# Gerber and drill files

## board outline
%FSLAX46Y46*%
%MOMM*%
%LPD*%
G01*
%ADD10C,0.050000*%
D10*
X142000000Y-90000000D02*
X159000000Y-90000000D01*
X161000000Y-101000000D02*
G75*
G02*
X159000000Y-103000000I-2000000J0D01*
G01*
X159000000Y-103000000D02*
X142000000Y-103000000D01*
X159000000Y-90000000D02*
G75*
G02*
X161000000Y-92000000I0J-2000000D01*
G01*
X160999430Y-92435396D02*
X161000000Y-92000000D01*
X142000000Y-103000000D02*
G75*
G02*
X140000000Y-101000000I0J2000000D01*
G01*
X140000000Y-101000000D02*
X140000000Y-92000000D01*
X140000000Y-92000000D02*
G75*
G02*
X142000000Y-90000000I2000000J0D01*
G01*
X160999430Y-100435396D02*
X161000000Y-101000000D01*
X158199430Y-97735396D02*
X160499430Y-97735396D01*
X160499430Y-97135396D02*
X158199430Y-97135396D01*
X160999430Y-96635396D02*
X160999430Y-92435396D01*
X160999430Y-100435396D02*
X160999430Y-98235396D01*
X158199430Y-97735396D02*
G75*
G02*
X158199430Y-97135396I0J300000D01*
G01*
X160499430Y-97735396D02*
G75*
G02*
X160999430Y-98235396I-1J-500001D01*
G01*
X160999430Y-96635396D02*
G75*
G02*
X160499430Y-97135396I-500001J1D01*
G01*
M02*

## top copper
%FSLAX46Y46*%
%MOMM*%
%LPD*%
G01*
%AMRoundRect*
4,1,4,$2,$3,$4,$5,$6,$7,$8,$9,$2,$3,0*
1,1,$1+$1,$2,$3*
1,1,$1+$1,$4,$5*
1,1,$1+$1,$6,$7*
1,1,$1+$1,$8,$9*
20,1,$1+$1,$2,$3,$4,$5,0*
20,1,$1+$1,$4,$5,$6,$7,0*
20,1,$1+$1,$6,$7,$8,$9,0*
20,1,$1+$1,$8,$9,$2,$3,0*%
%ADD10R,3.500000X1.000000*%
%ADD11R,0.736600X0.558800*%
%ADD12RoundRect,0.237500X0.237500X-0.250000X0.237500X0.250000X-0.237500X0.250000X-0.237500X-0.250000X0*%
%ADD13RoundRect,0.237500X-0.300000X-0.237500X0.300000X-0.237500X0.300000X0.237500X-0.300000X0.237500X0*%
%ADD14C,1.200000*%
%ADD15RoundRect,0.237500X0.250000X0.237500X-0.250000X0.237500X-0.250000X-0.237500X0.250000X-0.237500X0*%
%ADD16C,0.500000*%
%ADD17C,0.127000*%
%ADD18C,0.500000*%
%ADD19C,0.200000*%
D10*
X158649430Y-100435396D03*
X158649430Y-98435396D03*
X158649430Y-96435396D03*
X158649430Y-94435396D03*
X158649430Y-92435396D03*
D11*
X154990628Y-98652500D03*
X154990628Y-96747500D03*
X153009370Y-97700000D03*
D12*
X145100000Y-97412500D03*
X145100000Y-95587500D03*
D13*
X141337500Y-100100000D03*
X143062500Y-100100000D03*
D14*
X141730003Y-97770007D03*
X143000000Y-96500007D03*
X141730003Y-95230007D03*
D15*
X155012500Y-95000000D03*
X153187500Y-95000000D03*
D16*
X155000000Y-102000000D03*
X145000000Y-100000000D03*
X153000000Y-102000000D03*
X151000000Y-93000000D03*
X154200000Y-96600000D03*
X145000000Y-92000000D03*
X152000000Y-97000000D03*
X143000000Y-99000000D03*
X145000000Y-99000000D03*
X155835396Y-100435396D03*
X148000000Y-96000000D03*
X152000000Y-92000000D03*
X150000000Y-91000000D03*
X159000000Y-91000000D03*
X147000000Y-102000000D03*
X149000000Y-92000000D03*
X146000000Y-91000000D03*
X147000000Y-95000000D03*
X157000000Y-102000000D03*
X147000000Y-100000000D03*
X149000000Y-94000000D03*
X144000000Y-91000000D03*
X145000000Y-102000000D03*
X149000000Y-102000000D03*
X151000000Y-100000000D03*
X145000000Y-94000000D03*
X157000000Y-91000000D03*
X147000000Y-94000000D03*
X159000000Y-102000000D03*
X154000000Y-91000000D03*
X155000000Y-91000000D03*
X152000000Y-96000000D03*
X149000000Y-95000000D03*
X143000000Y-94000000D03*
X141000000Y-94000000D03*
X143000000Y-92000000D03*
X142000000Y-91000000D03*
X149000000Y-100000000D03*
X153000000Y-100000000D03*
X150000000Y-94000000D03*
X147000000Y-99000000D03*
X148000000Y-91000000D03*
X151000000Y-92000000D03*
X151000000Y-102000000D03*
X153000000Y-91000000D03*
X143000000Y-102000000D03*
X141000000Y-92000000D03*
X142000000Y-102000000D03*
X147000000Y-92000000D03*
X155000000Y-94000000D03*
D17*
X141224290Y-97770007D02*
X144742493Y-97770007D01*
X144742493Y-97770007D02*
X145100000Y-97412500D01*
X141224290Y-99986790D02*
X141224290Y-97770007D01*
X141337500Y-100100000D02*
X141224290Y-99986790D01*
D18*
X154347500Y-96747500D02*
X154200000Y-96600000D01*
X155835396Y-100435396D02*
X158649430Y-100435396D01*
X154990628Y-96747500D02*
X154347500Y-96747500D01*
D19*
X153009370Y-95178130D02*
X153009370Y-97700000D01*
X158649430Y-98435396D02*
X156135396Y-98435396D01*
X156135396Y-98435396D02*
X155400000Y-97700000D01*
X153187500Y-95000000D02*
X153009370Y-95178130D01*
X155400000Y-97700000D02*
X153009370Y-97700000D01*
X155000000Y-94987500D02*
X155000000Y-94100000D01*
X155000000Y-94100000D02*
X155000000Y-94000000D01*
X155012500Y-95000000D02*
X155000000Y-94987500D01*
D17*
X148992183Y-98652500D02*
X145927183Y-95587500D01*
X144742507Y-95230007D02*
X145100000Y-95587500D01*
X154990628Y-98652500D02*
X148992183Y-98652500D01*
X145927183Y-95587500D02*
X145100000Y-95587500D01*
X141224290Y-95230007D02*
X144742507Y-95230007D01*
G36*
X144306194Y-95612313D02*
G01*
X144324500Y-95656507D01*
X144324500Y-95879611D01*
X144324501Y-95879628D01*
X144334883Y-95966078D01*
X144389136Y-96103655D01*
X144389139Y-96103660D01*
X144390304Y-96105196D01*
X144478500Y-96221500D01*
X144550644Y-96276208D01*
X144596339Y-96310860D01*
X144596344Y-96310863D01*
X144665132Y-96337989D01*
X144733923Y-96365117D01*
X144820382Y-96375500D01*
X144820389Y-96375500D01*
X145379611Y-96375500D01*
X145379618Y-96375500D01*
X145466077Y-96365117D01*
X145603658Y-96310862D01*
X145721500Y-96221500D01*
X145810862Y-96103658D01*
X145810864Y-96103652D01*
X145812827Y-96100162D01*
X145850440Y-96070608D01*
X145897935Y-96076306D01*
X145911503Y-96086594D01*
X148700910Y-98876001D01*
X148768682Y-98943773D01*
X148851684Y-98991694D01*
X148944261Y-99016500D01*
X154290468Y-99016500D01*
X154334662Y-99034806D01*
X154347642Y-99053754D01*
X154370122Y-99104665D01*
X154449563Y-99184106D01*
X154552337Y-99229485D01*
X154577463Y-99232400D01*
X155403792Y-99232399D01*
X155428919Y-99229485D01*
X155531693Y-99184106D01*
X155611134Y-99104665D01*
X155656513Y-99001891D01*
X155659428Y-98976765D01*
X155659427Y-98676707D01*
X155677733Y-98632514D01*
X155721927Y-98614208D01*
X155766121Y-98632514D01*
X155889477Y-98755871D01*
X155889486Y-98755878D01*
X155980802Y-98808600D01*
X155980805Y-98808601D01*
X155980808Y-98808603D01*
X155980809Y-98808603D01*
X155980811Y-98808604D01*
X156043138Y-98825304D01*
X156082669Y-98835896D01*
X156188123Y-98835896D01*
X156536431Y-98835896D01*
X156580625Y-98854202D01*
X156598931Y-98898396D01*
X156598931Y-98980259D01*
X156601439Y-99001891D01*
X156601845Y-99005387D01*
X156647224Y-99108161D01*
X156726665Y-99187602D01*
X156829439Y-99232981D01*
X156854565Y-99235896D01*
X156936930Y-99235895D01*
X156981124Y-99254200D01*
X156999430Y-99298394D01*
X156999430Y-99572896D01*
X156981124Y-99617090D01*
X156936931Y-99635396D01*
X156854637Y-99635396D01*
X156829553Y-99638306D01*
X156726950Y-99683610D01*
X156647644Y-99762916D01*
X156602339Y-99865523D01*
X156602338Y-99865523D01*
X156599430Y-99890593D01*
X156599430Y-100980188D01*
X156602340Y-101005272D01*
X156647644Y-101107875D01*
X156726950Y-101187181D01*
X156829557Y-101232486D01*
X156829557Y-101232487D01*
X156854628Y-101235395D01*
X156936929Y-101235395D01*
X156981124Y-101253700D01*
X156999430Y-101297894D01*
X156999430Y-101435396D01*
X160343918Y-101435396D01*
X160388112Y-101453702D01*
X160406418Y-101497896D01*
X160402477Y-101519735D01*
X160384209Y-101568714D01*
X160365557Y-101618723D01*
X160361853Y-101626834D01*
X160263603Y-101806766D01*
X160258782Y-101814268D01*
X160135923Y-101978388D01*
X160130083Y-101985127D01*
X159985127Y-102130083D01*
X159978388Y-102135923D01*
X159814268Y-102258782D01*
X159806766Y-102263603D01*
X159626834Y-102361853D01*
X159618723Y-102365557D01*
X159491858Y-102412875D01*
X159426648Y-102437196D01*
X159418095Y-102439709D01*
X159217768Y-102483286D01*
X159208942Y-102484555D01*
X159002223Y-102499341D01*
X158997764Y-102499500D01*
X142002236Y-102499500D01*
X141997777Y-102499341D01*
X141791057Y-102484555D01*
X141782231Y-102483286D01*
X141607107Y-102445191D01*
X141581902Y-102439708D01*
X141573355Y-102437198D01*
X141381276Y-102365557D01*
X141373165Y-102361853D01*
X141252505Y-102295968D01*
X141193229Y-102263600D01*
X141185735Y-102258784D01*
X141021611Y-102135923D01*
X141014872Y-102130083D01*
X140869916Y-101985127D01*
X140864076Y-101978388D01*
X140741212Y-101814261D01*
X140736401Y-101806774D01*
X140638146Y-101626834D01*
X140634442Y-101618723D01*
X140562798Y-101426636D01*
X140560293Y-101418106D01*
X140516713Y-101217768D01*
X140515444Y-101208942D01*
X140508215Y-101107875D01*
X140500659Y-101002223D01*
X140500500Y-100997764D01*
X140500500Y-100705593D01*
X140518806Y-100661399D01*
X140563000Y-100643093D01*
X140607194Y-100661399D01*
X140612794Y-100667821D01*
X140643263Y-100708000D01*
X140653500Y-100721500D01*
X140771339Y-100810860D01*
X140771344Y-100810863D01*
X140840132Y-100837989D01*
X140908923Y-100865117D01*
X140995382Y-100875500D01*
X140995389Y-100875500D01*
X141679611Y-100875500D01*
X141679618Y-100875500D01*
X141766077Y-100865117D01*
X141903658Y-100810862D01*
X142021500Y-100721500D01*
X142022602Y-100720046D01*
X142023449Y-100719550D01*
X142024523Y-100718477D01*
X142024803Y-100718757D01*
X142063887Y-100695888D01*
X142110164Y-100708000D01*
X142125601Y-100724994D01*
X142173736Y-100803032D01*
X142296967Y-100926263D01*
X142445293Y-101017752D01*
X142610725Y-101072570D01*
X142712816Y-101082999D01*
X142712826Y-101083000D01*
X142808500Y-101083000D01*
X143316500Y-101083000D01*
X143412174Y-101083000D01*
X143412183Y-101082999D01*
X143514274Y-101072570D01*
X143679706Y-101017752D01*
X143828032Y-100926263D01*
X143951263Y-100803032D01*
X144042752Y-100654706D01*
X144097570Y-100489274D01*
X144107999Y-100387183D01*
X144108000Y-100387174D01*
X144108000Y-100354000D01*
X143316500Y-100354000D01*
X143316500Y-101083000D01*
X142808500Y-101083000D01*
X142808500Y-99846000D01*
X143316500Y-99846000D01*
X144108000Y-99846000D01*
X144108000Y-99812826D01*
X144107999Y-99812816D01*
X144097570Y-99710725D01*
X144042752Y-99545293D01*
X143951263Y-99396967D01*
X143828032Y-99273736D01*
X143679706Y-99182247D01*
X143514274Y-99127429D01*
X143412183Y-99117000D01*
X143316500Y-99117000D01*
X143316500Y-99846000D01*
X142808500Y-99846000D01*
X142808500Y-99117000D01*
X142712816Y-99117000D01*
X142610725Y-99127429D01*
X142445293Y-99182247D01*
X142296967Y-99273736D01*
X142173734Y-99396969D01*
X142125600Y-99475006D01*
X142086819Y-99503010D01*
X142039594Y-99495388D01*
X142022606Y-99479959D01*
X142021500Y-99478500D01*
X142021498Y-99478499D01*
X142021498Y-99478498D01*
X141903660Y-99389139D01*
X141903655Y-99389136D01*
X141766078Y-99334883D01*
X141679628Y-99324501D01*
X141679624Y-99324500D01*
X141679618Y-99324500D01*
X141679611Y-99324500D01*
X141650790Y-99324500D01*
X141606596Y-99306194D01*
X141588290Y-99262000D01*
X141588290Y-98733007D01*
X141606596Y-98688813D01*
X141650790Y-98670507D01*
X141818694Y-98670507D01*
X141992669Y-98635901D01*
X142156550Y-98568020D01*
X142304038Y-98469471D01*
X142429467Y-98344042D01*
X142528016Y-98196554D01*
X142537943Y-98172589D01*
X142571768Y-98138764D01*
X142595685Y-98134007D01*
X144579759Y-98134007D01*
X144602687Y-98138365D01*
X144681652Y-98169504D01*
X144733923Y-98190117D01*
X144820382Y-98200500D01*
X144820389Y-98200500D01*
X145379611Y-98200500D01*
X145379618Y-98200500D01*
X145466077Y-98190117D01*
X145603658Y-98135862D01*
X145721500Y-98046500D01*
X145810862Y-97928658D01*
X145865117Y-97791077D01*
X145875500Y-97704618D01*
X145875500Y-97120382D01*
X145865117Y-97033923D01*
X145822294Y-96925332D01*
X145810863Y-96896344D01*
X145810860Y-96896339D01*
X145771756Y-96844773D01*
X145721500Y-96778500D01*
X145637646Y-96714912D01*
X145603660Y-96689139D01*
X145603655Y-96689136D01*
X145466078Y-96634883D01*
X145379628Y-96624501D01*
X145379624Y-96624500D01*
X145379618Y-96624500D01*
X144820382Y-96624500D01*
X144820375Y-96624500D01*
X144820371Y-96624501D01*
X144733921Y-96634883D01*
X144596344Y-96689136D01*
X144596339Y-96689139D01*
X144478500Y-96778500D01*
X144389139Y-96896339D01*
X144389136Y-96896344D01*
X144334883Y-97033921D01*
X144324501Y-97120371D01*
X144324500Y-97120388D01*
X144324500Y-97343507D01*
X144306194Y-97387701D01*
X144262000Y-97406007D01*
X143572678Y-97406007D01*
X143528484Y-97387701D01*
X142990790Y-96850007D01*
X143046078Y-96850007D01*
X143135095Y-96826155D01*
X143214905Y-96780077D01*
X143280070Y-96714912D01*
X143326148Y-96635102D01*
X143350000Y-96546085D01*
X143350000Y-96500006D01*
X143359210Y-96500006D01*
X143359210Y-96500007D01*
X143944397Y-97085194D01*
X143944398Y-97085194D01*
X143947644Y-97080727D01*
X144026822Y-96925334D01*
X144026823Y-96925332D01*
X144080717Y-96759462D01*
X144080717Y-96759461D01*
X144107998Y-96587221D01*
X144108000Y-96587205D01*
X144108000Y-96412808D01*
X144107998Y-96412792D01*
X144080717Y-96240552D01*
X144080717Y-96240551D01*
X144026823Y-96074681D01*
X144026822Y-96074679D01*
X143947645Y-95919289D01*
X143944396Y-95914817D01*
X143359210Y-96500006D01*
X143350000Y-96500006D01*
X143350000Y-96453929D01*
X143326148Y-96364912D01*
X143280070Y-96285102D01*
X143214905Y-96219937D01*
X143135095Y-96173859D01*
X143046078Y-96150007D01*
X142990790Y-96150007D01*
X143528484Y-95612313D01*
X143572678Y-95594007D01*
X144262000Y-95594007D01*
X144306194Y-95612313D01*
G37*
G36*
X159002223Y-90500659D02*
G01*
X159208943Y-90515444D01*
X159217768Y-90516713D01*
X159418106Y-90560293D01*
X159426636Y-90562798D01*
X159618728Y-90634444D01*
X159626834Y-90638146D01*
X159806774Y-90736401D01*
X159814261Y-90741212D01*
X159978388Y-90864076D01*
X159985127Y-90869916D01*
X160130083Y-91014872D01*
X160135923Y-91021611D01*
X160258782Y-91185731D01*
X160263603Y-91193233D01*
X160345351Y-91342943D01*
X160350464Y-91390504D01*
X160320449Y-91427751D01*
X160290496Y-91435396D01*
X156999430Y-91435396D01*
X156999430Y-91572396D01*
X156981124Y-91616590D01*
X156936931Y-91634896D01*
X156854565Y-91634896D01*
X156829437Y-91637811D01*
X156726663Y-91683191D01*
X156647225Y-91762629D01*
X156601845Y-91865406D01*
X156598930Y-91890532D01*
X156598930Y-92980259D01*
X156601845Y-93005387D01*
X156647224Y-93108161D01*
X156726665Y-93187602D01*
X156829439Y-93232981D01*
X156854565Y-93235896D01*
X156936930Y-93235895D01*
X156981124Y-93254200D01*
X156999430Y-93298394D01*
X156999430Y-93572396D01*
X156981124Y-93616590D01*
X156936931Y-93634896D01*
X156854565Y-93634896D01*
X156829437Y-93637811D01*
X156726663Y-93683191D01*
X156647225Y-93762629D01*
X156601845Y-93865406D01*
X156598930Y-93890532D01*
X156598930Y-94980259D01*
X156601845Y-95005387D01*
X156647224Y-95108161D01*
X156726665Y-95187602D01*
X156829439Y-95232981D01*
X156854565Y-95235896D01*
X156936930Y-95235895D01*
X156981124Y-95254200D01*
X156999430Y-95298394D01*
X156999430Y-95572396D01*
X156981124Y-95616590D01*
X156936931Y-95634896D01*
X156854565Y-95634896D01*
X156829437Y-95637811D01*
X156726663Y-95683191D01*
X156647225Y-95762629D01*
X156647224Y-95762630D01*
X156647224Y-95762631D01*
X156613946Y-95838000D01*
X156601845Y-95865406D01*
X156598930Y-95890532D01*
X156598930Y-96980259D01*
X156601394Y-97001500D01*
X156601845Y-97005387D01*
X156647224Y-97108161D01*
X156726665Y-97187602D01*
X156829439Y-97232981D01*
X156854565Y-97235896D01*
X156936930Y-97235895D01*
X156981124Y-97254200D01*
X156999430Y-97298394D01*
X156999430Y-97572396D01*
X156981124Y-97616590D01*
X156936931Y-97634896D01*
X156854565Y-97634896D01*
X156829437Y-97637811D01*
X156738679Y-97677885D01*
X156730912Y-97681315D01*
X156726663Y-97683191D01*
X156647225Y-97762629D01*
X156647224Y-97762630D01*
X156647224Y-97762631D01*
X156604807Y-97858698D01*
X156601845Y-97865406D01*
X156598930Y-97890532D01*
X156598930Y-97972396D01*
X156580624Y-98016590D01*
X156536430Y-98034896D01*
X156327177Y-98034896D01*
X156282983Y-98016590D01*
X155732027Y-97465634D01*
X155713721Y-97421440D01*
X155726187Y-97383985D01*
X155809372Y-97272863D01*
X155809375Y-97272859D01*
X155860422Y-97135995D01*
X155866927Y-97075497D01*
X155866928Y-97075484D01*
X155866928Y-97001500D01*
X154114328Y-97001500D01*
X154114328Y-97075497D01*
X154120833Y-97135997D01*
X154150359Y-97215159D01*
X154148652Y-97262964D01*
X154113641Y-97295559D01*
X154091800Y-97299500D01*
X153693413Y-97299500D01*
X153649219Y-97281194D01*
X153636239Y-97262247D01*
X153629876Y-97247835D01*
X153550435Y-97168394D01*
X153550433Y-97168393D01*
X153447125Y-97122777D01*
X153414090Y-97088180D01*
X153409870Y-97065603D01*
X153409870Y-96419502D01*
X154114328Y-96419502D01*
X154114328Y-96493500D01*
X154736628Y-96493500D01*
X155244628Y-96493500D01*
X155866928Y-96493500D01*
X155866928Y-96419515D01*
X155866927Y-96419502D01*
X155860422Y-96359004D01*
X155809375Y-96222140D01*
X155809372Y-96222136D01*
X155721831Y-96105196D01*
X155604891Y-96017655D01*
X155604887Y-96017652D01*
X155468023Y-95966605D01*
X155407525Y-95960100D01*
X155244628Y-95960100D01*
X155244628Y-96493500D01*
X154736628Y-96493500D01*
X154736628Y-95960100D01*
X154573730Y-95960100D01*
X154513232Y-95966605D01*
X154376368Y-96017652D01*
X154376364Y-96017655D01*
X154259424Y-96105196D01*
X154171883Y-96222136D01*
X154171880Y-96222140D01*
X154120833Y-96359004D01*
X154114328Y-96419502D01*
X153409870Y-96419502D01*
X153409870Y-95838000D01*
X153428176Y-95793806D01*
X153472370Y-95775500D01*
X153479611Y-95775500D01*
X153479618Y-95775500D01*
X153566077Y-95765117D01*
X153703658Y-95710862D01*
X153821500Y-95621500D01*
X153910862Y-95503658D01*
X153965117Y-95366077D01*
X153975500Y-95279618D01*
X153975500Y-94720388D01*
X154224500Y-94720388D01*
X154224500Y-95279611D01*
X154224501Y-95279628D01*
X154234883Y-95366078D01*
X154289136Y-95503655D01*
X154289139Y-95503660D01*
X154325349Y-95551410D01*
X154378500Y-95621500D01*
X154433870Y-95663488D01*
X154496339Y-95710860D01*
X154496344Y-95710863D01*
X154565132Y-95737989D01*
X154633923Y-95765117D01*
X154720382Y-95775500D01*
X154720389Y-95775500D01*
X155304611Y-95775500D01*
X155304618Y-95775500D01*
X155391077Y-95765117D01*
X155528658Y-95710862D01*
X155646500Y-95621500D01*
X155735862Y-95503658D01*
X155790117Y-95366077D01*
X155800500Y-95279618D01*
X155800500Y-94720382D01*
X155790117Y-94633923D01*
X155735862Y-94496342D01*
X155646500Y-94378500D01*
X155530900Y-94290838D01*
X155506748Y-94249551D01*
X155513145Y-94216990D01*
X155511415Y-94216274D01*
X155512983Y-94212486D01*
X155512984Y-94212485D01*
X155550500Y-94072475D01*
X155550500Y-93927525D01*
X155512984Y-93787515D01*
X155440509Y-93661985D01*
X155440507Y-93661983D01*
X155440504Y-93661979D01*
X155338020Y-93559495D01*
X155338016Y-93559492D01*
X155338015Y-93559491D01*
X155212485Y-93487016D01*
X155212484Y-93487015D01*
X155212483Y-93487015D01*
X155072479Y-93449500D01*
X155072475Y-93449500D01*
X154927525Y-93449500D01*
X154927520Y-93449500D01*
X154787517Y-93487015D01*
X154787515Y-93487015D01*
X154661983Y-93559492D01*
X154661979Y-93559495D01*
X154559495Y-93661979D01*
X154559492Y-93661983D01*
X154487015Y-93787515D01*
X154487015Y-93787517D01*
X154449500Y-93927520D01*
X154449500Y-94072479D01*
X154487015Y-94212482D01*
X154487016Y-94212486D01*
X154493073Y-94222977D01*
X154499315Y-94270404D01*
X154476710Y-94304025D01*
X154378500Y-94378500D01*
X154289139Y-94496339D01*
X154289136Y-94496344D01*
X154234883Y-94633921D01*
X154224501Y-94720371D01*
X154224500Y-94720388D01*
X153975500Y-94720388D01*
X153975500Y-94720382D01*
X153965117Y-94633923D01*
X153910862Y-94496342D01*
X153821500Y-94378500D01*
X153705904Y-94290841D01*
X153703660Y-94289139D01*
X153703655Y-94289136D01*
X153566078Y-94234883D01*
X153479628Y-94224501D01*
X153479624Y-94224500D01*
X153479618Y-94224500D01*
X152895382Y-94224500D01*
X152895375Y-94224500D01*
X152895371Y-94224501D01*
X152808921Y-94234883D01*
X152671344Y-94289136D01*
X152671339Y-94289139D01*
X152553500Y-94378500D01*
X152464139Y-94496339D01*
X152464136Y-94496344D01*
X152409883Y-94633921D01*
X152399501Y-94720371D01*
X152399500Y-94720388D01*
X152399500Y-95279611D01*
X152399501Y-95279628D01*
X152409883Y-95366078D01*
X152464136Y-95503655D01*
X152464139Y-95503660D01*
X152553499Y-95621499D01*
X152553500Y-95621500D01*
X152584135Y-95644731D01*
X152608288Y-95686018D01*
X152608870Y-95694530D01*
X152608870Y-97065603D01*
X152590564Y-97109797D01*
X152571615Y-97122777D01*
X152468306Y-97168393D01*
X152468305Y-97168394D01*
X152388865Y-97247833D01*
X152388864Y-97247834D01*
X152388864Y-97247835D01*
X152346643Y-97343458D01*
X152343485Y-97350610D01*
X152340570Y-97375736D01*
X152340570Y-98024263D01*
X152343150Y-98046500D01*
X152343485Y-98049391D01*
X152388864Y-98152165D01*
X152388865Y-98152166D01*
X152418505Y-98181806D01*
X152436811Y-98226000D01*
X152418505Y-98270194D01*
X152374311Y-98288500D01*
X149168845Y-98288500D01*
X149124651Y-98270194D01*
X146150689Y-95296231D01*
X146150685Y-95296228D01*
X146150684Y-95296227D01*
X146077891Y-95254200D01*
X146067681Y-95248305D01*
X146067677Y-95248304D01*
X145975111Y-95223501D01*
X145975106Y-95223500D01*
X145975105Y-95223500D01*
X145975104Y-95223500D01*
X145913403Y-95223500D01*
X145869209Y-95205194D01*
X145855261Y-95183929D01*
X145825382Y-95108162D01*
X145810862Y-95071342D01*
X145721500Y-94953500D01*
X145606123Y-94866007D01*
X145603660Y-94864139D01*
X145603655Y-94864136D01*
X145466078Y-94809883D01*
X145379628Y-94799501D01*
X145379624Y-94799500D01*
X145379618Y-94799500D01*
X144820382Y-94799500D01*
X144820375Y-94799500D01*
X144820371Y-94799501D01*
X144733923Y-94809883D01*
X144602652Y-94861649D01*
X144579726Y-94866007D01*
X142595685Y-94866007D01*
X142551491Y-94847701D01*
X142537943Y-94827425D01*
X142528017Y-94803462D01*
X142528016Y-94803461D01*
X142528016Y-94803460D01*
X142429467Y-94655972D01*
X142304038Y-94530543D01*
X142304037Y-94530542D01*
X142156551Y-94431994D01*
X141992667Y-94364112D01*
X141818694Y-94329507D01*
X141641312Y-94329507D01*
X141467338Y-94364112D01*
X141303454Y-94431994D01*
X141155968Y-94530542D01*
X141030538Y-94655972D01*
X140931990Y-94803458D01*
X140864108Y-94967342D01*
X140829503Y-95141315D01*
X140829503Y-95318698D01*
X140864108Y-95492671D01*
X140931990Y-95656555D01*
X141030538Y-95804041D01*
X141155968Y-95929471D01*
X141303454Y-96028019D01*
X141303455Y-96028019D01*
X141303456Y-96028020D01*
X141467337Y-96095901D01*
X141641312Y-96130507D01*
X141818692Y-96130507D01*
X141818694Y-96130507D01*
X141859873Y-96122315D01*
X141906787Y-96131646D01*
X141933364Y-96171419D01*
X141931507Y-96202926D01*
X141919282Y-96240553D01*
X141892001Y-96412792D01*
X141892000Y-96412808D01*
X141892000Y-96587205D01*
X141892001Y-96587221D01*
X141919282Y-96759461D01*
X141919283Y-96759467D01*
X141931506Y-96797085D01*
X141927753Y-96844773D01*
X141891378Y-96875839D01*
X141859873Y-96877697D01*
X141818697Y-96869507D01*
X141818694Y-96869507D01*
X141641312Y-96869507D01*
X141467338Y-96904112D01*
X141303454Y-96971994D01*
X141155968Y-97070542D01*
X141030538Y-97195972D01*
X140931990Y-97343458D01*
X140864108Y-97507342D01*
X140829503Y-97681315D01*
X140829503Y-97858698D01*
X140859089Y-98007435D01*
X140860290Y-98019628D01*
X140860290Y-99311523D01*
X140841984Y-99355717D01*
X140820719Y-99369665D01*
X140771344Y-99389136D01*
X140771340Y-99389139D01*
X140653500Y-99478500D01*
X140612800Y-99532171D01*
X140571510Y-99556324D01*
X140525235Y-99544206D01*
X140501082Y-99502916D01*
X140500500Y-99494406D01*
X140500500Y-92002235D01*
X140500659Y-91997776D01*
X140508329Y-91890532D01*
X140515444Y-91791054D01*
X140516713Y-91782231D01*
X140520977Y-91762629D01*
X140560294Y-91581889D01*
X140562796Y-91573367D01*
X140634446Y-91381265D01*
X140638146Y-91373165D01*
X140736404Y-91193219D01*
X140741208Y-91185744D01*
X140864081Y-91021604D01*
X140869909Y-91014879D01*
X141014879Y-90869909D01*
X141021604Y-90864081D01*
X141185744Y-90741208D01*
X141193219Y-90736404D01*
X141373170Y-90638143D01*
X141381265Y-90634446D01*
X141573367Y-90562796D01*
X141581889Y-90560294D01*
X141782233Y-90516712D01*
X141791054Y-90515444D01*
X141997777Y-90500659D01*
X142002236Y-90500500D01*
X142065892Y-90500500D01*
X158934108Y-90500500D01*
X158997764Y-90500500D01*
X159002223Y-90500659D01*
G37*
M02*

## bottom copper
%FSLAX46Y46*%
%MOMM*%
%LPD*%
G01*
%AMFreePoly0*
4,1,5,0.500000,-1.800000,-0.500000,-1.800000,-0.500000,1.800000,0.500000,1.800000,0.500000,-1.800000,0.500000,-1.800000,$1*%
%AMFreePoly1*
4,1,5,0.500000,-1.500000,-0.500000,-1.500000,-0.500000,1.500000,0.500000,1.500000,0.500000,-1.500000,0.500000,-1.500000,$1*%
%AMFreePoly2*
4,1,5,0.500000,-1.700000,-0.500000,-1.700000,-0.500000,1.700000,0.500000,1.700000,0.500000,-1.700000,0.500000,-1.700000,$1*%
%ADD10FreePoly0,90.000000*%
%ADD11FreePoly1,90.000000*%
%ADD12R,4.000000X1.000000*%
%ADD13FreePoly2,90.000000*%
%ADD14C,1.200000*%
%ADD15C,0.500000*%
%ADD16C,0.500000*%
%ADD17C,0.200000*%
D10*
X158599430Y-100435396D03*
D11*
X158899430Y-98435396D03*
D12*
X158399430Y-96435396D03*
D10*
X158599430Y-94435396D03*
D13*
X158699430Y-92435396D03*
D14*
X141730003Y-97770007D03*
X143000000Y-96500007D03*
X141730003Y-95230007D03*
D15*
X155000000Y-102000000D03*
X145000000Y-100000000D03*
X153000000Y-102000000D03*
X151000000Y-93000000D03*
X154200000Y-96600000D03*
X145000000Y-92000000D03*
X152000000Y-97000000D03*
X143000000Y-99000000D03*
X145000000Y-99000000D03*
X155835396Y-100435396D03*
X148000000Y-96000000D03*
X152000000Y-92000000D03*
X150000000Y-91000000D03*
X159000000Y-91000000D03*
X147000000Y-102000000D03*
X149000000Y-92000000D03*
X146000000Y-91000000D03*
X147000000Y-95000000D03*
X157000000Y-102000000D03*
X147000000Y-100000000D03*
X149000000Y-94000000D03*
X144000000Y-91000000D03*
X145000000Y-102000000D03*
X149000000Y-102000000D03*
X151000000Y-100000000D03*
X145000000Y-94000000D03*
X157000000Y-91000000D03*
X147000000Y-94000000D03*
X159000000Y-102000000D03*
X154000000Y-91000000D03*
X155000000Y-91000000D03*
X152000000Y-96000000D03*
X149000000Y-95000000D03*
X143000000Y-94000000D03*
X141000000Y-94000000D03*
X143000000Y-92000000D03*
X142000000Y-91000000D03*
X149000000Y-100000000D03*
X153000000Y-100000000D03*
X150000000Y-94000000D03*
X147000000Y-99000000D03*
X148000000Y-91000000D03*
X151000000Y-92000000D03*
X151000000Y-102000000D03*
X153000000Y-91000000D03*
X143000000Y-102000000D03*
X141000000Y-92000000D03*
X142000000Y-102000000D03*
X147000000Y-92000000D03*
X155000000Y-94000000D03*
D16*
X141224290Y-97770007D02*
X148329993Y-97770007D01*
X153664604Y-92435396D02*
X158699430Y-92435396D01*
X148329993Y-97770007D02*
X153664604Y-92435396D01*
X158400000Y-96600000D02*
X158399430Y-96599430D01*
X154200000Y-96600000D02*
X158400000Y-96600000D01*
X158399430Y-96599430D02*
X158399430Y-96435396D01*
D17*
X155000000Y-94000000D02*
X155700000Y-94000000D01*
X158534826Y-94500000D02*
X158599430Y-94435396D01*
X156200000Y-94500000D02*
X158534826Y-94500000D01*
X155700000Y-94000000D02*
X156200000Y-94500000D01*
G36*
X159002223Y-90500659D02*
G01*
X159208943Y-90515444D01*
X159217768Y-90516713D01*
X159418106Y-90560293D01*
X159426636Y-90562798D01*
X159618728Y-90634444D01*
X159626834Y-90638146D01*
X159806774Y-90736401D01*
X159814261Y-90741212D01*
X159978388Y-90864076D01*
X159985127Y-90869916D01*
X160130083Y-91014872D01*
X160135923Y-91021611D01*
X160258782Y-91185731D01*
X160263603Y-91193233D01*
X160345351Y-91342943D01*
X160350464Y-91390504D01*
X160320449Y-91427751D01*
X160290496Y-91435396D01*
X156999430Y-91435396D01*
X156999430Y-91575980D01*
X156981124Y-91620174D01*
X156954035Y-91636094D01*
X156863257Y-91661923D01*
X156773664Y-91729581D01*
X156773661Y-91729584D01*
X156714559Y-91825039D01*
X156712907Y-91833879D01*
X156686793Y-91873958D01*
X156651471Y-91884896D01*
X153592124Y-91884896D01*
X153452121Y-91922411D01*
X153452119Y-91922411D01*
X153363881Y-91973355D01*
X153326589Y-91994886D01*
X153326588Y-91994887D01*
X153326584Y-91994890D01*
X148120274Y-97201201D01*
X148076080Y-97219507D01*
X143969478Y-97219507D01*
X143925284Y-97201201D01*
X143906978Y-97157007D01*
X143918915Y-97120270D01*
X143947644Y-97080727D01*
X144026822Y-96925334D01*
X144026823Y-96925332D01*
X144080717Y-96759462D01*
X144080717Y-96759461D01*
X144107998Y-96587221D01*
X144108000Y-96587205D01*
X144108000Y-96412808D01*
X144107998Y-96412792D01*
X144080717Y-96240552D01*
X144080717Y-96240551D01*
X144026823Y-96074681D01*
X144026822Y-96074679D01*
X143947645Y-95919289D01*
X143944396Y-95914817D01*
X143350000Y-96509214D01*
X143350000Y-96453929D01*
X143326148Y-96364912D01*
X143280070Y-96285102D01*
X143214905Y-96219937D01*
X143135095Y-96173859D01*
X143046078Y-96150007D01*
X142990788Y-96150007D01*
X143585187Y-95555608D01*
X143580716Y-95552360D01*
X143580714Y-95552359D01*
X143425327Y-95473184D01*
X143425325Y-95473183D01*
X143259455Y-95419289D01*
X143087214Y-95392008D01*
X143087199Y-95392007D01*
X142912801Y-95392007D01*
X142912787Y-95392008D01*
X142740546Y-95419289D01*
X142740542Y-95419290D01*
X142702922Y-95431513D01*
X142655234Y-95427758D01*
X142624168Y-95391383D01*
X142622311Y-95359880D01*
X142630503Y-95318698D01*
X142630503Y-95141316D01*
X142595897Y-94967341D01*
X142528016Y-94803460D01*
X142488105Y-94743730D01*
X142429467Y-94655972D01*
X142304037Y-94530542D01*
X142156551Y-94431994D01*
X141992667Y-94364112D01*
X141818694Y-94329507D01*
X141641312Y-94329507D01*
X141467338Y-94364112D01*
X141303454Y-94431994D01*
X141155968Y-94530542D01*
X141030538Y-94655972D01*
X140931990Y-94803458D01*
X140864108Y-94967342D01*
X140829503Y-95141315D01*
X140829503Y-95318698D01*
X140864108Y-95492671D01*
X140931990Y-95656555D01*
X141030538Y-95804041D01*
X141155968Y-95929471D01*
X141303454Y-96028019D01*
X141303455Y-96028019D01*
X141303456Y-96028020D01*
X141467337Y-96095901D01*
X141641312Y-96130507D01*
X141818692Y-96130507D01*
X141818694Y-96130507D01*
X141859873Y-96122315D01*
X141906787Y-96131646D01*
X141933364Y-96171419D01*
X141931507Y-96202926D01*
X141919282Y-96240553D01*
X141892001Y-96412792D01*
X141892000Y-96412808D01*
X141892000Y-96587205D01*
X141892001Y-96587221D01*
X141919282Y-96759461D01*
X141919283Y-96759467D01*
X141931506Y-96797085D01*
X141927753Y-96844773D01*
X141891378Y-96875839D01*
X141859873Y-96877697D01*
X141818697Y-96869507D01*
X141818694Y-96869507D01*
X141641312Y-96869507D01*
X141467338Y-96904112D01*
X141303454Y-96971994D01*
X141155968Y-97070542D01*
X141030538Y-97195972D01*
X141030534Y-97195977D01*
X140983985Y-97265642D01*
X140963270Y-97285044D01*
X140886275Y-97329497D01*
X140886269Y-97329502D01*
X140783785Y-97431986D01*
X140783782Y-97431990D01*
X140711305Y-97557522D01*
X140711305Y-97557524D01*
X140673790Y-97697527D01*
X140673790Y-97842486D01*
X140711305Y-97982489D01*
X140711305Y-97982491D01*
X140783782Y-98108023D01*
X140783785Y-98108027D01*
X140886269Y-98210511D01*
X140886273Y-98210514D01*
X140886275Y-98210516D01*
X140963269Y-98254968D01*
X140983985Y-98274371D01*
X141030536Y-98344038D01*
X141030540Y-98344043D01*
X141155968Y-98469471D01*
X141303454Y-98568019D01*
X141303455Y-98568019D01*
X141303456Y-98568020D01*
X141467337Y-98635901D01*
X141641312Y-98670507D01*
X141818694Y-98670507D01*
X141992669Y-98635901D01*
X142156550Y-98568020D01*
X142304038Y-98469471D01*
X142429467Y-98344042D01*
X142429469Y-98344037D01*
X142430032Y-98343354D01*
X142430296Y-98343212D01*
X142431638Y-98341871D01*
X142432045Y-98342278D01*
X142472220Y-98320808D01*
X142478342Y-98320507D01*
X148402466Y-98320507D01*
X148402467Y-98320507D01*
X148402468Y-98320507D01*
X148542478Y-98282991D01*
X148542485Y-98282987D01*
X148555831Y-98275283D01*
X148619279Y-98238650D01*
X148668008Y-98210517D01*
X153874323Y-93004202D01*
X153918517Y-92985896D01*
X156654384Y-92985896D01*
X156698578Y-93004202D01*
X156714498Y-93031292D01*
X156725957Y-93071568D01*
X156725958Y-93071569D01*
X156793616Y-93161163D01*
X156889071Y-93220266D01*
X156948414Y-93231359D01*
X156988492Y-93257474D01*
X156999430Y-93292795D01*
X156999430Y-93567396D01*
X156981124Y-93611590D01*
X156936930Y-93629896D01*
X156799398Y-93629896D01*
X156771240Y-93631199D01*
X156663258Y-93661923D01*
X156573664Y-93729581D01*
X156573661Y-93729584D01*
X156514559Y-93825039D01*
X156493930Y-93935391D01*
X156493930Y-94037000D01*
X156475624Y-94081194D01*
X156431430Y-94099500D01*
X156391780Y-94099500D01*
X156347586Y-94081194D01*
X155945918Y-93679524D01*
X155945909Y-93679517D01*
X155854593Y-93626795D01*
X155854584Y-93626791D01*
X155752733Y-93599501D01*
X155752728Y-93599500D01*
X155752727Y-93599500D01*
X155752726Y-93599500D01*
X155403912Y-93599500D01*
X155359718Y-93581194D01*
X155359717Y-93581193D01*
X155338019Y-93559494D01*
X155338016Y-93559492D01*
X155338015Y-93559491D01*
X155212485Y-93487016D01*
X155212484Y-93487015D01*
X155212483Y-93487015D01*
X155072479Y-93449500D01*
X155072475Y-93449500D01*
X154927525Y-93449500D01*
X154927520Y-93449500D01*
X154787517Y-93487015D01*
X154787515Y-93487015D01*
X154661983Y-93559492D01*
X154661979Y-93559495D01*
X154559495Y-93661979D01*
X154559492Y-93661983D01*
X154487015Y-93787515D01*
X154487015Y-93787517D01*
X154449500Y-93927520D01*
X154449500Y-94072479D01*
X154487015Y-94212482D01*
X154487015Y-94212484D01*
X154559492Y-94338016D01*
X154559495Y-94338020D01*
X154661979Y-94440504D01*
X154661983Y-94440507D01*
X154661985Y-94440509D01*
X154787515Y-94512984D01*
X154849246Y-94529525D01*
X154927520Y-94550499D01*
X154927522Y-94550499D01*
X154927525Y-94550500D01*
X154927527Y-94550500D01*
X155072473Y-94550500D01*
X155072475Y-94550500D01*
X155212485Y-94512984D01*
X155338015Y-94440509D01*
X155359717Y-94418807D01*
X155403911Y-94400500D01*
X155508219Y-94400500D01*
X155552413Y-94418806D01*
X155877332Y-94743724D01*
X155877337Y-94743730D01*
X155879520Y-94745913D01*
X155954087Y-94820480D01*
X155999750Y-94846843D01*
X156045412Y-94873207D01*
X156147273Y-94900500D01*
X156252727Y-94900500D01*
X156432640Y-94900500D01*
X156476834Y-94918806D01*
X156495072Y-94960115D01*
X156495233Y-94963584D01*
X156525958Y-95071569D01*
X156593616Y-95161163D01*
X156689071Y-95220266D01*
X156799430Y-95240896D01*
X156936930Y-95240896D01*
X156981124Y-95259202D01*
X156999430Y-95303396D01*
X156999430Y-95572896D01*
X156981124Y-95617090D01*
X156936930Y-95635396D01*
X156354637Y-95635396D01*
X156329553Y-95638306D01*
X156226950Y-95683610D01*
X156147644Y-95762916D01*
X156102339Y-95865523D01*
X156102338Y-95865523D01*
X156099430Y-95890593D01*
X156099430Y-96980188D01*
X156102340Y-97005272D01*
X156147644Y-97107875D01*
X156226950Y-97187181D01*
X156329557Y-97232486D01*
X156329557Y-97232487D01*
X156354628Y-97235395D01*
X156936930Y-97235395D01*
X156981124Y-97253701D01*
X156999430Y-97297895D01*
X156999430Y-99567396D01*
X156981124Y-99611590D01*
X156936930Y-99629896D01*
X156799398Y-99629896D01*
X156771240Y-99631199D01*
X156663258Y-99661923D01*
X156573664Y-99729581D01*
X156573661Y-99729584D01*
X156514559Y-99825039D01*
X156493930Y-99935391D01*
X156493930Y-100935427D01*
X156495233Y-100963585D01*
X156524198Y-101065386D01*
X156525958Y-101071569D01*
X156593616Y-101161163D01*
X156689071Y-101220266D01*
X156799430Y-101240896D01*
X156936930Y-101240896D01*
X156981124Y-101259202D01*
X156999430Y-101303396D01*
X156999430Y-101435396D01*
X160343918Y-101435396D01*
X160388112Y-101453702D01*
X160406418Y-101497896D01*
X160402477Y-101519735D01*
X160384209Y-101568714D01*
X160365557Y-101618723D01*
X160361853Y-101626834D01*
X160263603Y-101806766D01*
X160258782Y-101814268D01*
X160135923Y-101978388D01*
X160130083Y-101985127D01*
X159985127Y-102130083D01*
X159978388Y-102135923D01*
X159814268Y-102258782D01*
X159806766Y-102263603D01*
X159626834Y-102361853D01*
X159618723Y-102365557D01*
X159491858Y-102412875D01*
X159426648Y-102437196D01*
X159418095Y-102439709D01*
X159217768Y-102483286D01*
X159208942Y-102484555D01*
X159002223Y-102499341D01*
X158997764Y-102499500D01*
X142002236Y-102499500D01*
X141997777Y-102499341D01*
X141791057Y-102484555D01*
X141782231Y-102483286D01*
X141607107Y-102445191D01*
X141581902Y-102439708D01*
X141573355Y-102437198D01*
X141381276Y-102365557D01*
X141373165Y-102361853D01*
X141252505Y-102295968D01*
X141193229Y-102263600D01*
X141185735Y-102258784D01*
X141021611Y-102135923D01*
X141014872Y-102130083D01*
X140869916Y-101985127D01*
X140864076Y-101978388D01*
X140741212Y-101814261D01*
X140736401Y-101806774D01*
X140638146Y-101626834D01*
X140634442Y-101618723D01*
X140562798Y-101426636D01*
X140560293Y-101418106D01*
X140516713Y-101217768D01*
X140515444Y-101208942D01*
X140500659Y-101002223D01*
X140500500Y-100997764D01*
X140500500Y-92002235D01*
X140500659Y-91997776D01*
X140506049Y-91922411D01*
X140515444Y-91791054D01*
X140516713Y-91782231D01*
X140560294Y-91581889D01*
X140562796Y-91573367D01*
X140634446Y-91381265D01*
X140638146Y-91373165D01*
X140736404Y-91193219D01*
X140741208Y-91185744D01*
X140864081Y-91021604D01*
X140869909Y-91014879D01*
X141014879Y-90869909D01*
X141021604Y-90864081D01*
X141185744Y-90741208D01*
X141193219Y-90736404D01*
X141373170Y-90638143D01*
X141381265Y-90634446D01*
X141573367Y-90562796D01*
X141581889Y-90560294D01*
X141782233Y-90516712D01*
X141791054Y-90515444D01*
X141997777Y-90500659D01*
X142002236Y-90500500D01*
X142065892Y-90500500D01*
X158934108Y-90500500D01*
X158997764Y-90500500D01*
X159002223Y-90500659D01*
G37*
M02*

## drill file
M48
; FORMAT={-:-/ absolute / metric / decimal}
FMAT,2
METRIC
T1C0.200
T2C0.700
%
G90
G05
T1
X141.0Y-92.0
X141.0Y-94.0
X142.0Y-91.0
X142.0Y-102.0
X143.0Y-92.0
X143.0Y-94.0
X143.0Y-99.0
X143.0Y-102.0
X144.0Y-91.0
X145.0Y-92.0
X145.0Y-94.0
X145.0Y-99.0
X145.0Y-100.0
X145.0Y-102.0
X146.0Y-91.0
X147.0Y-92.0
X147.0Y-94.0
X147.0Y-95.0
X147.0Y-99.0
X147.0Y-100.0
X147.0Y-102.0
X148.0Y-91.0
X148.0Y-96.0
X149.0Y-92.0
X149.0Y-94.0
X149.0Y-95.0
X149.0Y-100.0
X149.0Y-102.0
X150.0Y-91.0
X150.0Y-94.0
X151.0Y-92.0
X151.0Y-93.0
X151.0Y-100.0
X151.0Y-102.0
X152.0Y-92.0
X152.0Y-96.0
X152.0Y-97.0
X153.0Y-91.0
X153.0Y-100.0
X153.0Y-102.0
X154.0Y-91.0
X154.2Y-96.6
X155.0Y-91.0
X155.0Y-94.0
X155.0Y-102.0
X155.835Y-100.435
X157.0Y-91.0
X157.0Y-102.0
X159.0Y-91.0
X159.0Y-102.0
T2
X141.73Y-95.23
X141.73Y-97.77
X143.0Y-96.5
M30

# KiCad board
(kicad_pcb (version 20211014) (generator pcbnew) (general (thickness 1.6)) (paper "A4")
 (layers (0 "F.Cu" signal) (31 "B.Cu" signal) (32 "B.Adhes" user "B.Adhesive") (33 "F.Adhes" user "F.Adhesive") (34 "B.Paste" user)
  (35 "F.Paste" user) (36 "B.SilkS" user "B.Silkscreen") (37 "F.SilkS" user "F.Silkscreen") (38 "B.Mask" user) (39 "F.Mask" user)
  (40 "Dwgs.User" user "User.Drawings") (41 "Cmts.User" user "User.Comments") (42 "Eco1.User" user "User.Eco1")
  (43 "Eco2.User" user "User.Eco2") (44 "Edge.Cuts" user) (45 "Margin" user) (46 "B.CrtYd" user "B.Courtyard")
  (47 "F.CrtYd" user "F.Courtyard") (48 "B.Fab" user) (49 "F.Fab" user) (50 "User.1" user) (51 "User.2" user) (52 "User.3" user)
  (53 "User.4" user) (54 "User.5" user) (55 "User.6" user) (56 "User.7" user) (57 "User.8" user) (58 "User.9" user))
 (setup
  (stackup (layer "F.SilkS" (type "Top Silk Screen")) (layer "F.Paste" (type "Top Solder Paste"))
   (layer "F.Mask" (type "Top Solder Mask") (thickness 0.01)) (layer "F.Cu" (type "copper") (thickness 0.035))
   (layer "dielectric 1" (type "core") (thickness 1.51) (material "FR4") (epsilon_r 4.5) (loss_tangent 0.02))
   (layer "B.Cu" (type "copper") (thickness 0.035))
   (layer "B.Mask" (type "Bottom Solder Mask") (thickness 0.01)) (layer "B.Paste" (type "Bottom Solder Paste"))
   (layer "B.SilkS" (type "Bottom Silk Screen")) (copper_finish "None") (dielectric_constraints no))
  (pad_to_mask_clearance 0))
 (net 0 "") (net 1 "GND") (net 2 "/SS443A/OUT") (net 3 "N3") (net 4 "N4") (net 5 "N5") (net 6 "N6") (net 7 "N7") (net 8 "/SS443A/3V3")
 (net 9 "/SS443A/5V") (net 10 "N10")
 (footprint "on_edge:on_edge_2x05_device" (layer "F.Cu") (at 160.99943 96.435396 90)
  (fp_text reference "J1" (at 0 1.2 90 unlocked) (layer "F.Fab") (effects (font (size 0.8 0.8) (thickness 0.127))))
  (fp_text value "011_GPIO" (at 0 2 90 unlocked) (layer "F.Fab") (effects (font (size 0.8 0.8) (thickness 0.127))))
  (fp_line (start -1.3 -2.8) (end -1.3 -0.5) (layer "Edge.Cuts") (width 0.05))
  (fp_line (start -0.7 -0.5) (end -0.7 -2.8) (layer "Edge.Cuts") (width 0.05))
  (fp_line (start -0.2 0) (end 4 0) (layer "Edge.Cuts") (width 0.05))
  (fp_line (start -4 0) (end -1.8 0) (layer "Edge.Cuts") (width 0.05))
  (fp_arc (start -1.3 -2.8) (mid -1 -3.1) (end -0.7 -2.8) (layer "Edge.Cuts") (width 0.05))
  (fp_arc (start -1.3 -0.5) (mid -1.446447 -0.146447) (end -1.8 0) (layer "Edge.Cuts") (width 0.05))
  (fp_arc (start -0.2 0) (mid -0.553553 -0.146447) (end -0.7 -0.5) (layer "Edge.Cuts") (width 0.05))
  (pad "1" smd rect (at -4 -2.35 270) (size 1 3.5) (layers "F.Cu" "F.Mask") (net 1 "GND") (zone_connect 0))
  (pad "2" smd rect (at -2 -2.35 90) (size 1 3.5) (layers "F.Cu" "F.Mask") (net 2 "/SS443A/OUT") (zone_connect 0))
  (pad "3" smd rect (at 0 -2.35 90) (size 1 3.5) (layers "F.Cu" "F.Mask") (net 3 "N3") (zone_connect 0))
  (pad "4" smd rect (at 2 -2.35 270) (size 1 3.5) (layers "F.Cu" "F.Mask") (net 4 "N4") (zone_connect 0))
  (pad "5" smd rect (at 4 -2.35 270) (size 1 3.5) (layers "F.Cu" "F.Mask") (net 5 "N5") (zone_connect 0))
  (pad "6" smd custom (at -4 -2.4 90) (size 1 3.6) (layers "B.Cu" "B.Mask") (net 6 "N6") (zone_connect 0)
   (options (clearance outline) (anchor rect)) (primitives))
  (pad "7" smd custom (at -2 -2.1 90) (size 1 3) (layers "B.Cu" "B.Mask") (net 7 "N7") (zone_connect 0)
   (options (clearance outline) (anchor rect)) (primitives))
  (pad "8" smd rect (at 0 -2.6 90) (size 1 4) (layers "B.Cu" "B.Mask") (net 1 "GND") (zone_connect 0))
  (pad "9" smd custom (at 2 -2.4 90) (size 1 3.6) (layers "B.Cu" "B.Mask") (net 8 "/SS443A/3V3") (zone_connect 0)
   (options (clearance outline) (anchor rect)) (primitives))
  (pad "10" smd custom (at 4 -2.3 90) (size 1 3.4) (layers "B.Cu" "B.Mask") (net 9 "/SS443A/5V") (zone_connect 0)
   (options (clearance outline) (anchor rect)) (primitives))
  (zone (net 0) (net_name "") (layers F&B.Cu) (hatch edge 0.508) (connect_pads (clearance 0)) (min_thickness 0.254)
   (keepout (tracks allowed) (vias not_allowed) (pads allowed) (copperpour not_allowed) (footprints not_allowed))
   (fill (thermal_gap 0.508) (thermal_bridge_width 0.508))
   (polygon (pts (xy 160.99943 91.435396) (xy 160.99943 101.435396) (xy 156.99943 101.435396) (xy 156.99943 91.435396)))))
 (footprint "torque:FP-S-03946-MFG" (layer "F.Cu") (at 154 97.7 180)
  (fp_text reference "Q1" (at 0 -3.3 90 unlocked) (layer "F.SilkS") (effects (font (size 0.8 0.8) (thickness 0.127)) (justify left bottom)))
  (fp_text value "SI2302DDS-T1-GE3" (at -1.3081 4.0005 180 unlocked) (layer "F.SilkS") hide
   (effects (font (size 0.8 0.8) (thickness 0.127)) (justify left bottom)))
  (pad "1" smd rect (at -0.990628 -0.9525 180) (size 0.7366 0.5588) (layers "F.Cu" "F.Paste" "F.Mask") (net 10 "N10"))
  (pad "2" smd rect (at -0.990628 0.9525 180) (size 0.7366 0.5588) (layers "F.Cu" "F.Paste" "F.Mask") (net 1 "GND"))
  (pad "3" smd rect (at 0.99063 0 180) (size 0.7366 0.5588) (layers "F.Cu" "F.Paste" "F.Mask") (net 2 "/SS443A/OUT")))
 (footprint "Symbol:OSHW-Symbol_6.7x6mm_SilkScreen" (layer "F.Cu") (at 149.1 99)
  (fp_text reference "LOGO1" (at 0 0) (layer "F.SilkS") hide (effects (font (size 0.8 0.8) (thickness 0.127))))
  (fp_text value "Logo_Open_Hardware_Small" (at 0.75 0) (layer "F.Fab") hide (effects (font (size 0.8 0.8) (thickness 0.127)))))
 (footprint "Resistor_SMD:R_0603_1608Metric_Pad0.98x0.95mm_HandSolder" (layer "F.Cu") (at 145.1 96.5 90)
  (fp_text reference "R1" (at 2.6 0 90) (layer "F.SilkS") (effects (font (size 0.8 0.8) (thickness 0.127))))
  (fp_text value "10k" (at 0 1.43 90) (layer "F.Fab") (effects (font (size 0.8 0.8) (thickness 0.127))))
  (pad "1" smd roundrect (at -0.9125 0 90) (size 0.975 0.95) (layers "F.Cu" "F.Paste" "F.Mask") (roundrect_rratio 0.25) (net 9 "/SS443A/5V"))
  (pad "2" smd roundrect (at 0.9125 0 90) (size 0.975 0.95) (layers "F.Cu" "F.Paste" "F.Mask") (roundrect_rratio 0.25) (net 10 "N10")))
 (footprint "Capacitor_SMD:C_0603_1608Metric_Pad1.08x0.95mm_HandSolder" (layer "F.Cu") (at 142.2 100.1)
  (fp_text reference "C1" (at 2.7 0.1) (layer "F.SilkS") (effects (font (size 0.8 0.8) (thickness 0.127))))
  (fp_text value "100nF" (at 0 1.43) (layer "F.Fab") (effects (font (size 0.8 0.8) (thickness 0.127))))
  (pad "1" smd roundrect (at -0.8625 0) (size 1.075 0.95) (layers "F.Cu" "F.Paste" "F.Mask") (roundrect_rratio 0.25) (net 9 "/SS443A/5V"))
  (pad "2" smd roundrect (at 0.8625 0) (size 1.075 0.95) (layers "F.Cu" "F.Paste" "F.Mask") (roundrect_rratio 0.25) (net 1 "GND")))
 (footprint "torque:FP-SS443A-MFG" (layer "F.Cu") (at 141.895 96.500007 180)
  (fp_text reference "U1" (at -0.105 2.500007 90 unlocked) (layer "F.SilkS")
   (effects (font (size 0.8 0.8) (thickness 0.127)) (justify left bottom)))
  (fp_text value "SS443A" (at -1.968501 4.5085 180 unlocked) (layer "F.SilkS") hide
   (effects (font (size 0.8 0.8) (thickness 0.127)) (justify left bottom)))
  (pad "1" thru_hole circle (at 0.164997 -1.27 180) (size 1.2 1.2) (drill 0.7) (layers *.Cu *.Mask) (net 9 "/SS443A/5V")
   (solder_paste_margin -1000))
  (pad "2" thru_hole circle (at -1.105 0 180) (size 1.2 1.2) (drill 0.7) (layers *.Cu *.Mask) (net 1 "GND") (solder_paste_margin -1000))
  (pad "3" thru_hole circle (at 0.164997 1.27 180) (size 1.2 1.2) (drill 0.7) (layers *.Cu *.Mask) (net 10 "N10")
   (solder_paste_margin -1000)))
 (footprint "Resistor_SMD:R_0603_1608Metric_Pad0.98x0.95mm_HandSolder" (layer "F.Cu") (at 154.1 95 180)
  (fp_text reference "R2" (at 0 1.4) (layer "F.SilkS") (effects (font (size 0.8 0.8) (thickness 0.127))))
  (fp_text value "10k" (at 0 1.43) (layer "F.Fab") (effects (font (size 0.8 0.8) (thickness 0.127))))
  (pad "1" smd roundrect (at -0.9125 0 180) (size 0.975 0.95) (layers "F.Cu" "F.Paste" "F.Mask") (roundrect_rratio 0.25)
   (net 8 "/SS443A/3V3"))
  (pad "2" smd roundrect (at 0.9125 0 180) (size 0.975 0.95) (layers "F.Cu" "F.Paste" "F.Mask") (roundrect_rratio 0.25)
   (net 2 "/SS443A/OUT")))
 (gr_line (start 142 90) (end 159 90) (layer "Edge.Cuts") (width 0.05))
 (gr_arc (start 161 101) (mid 160.414214 102.414214) (end 159 103) (layer "Edge.Cuts") (width 0.05))
 (gr_line (start 159 103) (end 142 103) (layer "Edge.Cuts") (width 0.05))
 (gr_arc (start 159 90) (mid 160.414214 90.585786) (end 161 92) (layer "Edge.Cuts") (width 0.05))
 (gr_line (start 160.99943 92.435396) (end 161 92) (layer "Edge.Cuts") (width 0.05))
 (gr_arc (start 142 103) (mid 140.585786 102.414214) (end 140 101) (layer "Edge.Cuts") (width 0.05))
 (gr_line (start 140 101) (end 140 92) (layer "Edge.Cuts") (width 0.05))
 (gr_arc (start 140 92) (mid 140.585786 90.585786) (end 142 90) (layer "Edge.Cuts") (width 0.05))
 (gr_line (start 160.99943 100.435396) (end 161 101) (layer "Edge.Cuts") (width 0.05))
 (segment (start 141.22429 97.770007) (end 144.742493 97.770007) (width 0.127) (layer "F.Cu") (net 9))
 (segment (start 144.742493 97.770007) (end 145.1 97.4125) (width 0.127) (layer "F.Cu") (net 9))
 (segment (start 141.22429 99.98679) (end 141.22429 97.770007) (width 0.127) (layer "F.Cu") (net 9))
 (segment (start 141.3375 100.1) (end 141.22429 99.98679) (width 0.127) (layer "F.Cu") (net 9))
 (segment (start 141.22429 97.770007) (end 148.329993 97.770007) (width 0.5) (layer "B.Cu") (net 9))
 (segment (start 153.664604 92.435396) (end 158.69943 92.435396) (width 0.5) (layer "B.Cu") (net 9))
 (segment (start 148.329993 97.770007) (end 153.664604 92.435396) (width 0.5) (layer "B.Cu") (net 9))
 (segment (start 154.3475 96.7475) (end 154.2 96.6) (width 0.5) (layer "F.Cu") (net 1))
 (segment (start 155.835396 100.435396) (end 158.64943 100.435396) (width 0.5) (layer "F.Cu") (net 1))
 (segment (start 154.990628 96.7475) (end 154.3475 96.7475) (width 0.5) (layer "F.Cu") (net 1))
 (via (at 155 102) (size 0.5) (drill 0.2) (layers "F.Cu" "B.Cu") (free) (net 1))
 (via (at 145 100) (size 0.5) (drill 0.2) (layers "F.Cu" "B.Cu") (free) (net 1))
 (via (at 153 102) (size 0.5) (drill 0.2) (layers "F.Cu" "B.Cu") (free) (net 1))
 (via (at 151 93) (size 0.5) (drill 0.2) (layers "F.Cu" "B.Cu") (free) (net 1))
 (via (at 154.2 96.6) (size 0.5) (drill 0.2) (layers "F.Cu" "B.Cu") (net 1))
 (via (at 145 92) (size 0.5) (drill 0.2) (layers "F.Cu" "B.Cu") (free) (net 1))
 (via (at 152 97) (size 0.5) (drill 0.2) (layers "F.Cu" "B.Cu") (free) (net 1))
 (via (at 143 99) (size 0.5) (drill 0.2) (layers "F.Cu" "B.Cu") (free) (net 1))
 (via (at 145 99) (size 0.5) (drill 0.2) (layers "F.Cu" "B.Cu") (free) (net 1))
 (via (at 155.835396 100.435396) (size 0.5) (drill 0.2) (layers "F.Cu" "B.Cu") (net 1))
 (via (at 148 96) (size 0.5) (drill 0.2) (layers "F.Cu" "B.Cu") (free) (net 1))
 (via (at 152 92) (size 0.5) (drill 0.2) (layers "F.Cu" "B.Cu") (free) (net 1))
 (via (at 150 91) (size 0.5) (drill 0.2) (layers "F.Cu" "B.Cu") (free) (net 1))
 (via (at 159 91) (size 0.5) (drill 0.2) (layers "F.Cu" "B.Cu") (free) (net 1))
 (via (at 147 102) (size 0.5) (drill 0.2) (layers "F.Cu" "B.Cu") (free) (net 1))
 (via (at 149 92) (size 0.5) (drill 0.2) (layers "F.Cu" "B.Cu") (free) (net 1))
 (via (at 146 91) (size 0.5) (drill 0.2) (layers "F.Cu" "B.Cu") (free) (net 1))
 (via (at 147 95) (size 0.5) (drill 0.2) (layers "F.Cu" "B.Cu") (free) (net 1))
 (via (at 157 102) (size 0.5) (drill 0.2) (layers "F.Cu" "B.Cu") (free) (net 1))
 (via (at 147 100) (size 0.5) (drill 0.2) (layers "F.Cu" "B.Cu") (free) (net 1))
 (via (at 149 94) (size 0.5) (drill 0.2) (layers "F.Cu" "B.Cu") (free) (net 1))
 (via (at 144 91) (size 0.5) (drill 0.2) (layers "F.Cu" "B.Cu") (free) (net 1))
 (via (at 145 102) (size 0.5) (drill 0.2) (layers "F.Cu" "B.Cu") (free) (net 1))
 (via (at 149 102) (size 0.5) (drill 0.2) (layers "F.Cu" "B.Cu") (free) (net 1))
 (via (at 151 100) (size 0.5) (drill 0.2) (layers "F.Cu" "B.Cu") (free) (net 1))
 (via (at 145 94) (size 0.5) (drill 0.2) (layers "F.Cu" "B.Cu") (free) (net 1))
 (via (at 157 91) (size 0.5) (drill 0.2) (layers "F.Cu" "B.Cu") (free) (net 1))
 (via (at 147 94) (size 0.5) (drill 0.2) (layers "F.Cu" "B.Cu") (free) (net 1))
 (via (at 159 102) (size 0.5) (drill 0.2) (layers "F.Cu" "B.Cu") (free) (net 1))
 (via (at 154 91) (size 0.5) (drill 0.2) (layers "F.Cu" "B.Cu") (free) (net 1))
 (via (at 155 91) (size 0.5) (drill 0.2) (layers "F.Cu" "B.Cu") (free) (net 1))
 (via (at 152 96) (size 0.5) (drill 0.2) (layers "F.Cu" "B.Cu") (free) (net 1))
 (via (at 149 95) (size 0.5) (drill 0.2) (layers "F.Cu" "B.Cu") (free) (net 1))
 (via (at 143 94) (size 0.5) (drill 0.2) (layers "F.Cu" "B.Cu") (free) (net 1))
 (via (at 141 94) (size 0.5) (drill 0.2) (layers "F.Cu" "B.Cu") (free) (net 1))
 (via (at 143 92) (size 0.5) (drill 0.2) (layers "F.Cu" "B.Cu") (free) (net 1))
 (via (at 142 91) (size 0.5) (drill 0.2) (layers "F.Cu" "B.Cu") (free) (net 1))
 (via (at 149 100) (size 0.5) (drill 0.2) (layers "F.Cu" "B.Cu") (free) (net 1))
 (via (at 153 100) (size 0.5) (drill 0.2) (layers "F.Cu" "B.Cu") (free) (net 1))
 (via (at 150 94) (size 0.5) (drill 0.2) (layers "F.Cu" "B.Cu") (free) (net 1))
 (via (at 147 99) (size 0.5) (drill 0.2) (layers "F.Cu" "B.Cu") (free) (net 1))
 (via (at 148 91) (size 0.5) (drill 0.2) (layers "F.Cu" "B.Cu") (free) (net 1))
 (via (at 151 92) (size 0.5) (drill 0.2) (layers "F.Cu" "B.Cu") (free) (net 1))
 (via (at 151 102) (size 0.5) (drill 0.2) (layers "F.Cu" "B.Cu") (free) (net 1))
 (via (at 153 91) (size 0.5) (drill 0.2) (layers "F.Cu" "B.Cu") (free) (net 1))
 (via (at 143 102) (size 0.5) (drill 0.2) (layers "F.Cu" "B.Cu") (free) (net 1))
 (via (at 141 92) (size 0.5) (drill 0.2) (layers "F.Cu" "B.Cu") (free) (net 1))
 (via (at 142 102) (size 0.5) (drill 0.2) (layers "F.Cu" "B.Cu") (free) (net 1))
 (via (at 147 92) (size 0.5) (drill 0.2) (layers "F.Cu" "B.Cu") (free) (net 1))
 (segment (start 158.4 96.6) (end 158.39943 96.59943) (width 0.5) (layer "B.Cu") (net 1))
 (segment (start 154.2 96.6) (end 158.4 96.6) (width 0.5) (layer "B.Cu") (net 1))
 (segment (start 158.39943 96.59943) (end 158.39943 96.435396) (width 0.5) (layer "B.Cu") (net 1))
 (segment (start 153.00937 95.17813) (end 153.00937 97.7) (width 0.2) (layer "F.Cu") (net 2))
 (segment (start 158.64943 98.435396) (end 156.135396 98.435396) (width 0.2) (layer "F.Cu") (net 2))
 (segment (start 156.135396 98.435396) (end 155.4 97.7) (width 0.2) (layer "F.Cu") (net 2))
 (segment (start 153.1875 95) (end 153.00937 95.17813) (width 0.2) (layer "F.Cu") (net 2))
 (segment (start 155.4 97.7) (end 153.00937 97.7) (width 0.2) (layer "F.Cu") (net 2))
 (segment (start 155 94.9875) (end 155 94.1) (width 0.2) (layer "F.Cu") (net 8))
 (segment (start 155 94.1) (end 155 94) (width 0.2) (layer "F.Cu") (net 8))
 (segment (start 155.0125 95) (end 155 94.9875) (width 0.2) (layer "F.Cu") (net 8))
 (via (at 155 94) (size 0.5) (drill 0.2) (layers "F.Cu" "B.Cu") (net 8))
 (segment (start 155 94) (end 155.7 94) (width 0.2) (layer "B.Cu") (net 8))
 (segment (start 158.534826 94.5) (end 158.59943 94.435396) (width 0.2) (layer "B.Cu") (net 8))
 (segment (start 156.2 94.5) (end 158.534826 94.5) (width 0.2) (layer "B.Cu") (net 8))
 (segment (start 155.7 94) (end 156.2 94.5) (width 0.2) (layer "B.Cu") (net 8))
 (segment (start 148.992183 98.6525) (end 145.927183 95.5875) (width 0.127) (layer "F.Cu") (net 10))
 (segment (start 144.742507 95.230007) (end 145.1 95.5875) (width 0.127) (layer "F.Cu") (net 10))
 (segment (start 154.990628 98.6525) (end 148.992183 98.6525) (width 0.127) (layer "F.Cu") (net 10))
 (segment (start 145.927183 95.5875) (end 145.1 95.5875) (width 0.127) (layer "F.Cu") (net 10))
 (segment (start 141.22429 95.230007) (end 144.742507 95.230007) (width 0.127) (layer "F.Cu") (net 10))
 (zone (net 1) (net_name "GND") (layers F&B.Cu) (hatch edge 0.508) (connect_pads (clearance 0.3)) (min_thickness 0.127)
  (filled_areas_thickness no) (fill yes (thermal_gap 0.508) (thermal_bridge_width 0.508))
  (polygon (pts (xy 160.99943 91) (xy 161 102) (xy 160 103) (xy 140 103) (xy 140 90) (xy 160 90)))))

